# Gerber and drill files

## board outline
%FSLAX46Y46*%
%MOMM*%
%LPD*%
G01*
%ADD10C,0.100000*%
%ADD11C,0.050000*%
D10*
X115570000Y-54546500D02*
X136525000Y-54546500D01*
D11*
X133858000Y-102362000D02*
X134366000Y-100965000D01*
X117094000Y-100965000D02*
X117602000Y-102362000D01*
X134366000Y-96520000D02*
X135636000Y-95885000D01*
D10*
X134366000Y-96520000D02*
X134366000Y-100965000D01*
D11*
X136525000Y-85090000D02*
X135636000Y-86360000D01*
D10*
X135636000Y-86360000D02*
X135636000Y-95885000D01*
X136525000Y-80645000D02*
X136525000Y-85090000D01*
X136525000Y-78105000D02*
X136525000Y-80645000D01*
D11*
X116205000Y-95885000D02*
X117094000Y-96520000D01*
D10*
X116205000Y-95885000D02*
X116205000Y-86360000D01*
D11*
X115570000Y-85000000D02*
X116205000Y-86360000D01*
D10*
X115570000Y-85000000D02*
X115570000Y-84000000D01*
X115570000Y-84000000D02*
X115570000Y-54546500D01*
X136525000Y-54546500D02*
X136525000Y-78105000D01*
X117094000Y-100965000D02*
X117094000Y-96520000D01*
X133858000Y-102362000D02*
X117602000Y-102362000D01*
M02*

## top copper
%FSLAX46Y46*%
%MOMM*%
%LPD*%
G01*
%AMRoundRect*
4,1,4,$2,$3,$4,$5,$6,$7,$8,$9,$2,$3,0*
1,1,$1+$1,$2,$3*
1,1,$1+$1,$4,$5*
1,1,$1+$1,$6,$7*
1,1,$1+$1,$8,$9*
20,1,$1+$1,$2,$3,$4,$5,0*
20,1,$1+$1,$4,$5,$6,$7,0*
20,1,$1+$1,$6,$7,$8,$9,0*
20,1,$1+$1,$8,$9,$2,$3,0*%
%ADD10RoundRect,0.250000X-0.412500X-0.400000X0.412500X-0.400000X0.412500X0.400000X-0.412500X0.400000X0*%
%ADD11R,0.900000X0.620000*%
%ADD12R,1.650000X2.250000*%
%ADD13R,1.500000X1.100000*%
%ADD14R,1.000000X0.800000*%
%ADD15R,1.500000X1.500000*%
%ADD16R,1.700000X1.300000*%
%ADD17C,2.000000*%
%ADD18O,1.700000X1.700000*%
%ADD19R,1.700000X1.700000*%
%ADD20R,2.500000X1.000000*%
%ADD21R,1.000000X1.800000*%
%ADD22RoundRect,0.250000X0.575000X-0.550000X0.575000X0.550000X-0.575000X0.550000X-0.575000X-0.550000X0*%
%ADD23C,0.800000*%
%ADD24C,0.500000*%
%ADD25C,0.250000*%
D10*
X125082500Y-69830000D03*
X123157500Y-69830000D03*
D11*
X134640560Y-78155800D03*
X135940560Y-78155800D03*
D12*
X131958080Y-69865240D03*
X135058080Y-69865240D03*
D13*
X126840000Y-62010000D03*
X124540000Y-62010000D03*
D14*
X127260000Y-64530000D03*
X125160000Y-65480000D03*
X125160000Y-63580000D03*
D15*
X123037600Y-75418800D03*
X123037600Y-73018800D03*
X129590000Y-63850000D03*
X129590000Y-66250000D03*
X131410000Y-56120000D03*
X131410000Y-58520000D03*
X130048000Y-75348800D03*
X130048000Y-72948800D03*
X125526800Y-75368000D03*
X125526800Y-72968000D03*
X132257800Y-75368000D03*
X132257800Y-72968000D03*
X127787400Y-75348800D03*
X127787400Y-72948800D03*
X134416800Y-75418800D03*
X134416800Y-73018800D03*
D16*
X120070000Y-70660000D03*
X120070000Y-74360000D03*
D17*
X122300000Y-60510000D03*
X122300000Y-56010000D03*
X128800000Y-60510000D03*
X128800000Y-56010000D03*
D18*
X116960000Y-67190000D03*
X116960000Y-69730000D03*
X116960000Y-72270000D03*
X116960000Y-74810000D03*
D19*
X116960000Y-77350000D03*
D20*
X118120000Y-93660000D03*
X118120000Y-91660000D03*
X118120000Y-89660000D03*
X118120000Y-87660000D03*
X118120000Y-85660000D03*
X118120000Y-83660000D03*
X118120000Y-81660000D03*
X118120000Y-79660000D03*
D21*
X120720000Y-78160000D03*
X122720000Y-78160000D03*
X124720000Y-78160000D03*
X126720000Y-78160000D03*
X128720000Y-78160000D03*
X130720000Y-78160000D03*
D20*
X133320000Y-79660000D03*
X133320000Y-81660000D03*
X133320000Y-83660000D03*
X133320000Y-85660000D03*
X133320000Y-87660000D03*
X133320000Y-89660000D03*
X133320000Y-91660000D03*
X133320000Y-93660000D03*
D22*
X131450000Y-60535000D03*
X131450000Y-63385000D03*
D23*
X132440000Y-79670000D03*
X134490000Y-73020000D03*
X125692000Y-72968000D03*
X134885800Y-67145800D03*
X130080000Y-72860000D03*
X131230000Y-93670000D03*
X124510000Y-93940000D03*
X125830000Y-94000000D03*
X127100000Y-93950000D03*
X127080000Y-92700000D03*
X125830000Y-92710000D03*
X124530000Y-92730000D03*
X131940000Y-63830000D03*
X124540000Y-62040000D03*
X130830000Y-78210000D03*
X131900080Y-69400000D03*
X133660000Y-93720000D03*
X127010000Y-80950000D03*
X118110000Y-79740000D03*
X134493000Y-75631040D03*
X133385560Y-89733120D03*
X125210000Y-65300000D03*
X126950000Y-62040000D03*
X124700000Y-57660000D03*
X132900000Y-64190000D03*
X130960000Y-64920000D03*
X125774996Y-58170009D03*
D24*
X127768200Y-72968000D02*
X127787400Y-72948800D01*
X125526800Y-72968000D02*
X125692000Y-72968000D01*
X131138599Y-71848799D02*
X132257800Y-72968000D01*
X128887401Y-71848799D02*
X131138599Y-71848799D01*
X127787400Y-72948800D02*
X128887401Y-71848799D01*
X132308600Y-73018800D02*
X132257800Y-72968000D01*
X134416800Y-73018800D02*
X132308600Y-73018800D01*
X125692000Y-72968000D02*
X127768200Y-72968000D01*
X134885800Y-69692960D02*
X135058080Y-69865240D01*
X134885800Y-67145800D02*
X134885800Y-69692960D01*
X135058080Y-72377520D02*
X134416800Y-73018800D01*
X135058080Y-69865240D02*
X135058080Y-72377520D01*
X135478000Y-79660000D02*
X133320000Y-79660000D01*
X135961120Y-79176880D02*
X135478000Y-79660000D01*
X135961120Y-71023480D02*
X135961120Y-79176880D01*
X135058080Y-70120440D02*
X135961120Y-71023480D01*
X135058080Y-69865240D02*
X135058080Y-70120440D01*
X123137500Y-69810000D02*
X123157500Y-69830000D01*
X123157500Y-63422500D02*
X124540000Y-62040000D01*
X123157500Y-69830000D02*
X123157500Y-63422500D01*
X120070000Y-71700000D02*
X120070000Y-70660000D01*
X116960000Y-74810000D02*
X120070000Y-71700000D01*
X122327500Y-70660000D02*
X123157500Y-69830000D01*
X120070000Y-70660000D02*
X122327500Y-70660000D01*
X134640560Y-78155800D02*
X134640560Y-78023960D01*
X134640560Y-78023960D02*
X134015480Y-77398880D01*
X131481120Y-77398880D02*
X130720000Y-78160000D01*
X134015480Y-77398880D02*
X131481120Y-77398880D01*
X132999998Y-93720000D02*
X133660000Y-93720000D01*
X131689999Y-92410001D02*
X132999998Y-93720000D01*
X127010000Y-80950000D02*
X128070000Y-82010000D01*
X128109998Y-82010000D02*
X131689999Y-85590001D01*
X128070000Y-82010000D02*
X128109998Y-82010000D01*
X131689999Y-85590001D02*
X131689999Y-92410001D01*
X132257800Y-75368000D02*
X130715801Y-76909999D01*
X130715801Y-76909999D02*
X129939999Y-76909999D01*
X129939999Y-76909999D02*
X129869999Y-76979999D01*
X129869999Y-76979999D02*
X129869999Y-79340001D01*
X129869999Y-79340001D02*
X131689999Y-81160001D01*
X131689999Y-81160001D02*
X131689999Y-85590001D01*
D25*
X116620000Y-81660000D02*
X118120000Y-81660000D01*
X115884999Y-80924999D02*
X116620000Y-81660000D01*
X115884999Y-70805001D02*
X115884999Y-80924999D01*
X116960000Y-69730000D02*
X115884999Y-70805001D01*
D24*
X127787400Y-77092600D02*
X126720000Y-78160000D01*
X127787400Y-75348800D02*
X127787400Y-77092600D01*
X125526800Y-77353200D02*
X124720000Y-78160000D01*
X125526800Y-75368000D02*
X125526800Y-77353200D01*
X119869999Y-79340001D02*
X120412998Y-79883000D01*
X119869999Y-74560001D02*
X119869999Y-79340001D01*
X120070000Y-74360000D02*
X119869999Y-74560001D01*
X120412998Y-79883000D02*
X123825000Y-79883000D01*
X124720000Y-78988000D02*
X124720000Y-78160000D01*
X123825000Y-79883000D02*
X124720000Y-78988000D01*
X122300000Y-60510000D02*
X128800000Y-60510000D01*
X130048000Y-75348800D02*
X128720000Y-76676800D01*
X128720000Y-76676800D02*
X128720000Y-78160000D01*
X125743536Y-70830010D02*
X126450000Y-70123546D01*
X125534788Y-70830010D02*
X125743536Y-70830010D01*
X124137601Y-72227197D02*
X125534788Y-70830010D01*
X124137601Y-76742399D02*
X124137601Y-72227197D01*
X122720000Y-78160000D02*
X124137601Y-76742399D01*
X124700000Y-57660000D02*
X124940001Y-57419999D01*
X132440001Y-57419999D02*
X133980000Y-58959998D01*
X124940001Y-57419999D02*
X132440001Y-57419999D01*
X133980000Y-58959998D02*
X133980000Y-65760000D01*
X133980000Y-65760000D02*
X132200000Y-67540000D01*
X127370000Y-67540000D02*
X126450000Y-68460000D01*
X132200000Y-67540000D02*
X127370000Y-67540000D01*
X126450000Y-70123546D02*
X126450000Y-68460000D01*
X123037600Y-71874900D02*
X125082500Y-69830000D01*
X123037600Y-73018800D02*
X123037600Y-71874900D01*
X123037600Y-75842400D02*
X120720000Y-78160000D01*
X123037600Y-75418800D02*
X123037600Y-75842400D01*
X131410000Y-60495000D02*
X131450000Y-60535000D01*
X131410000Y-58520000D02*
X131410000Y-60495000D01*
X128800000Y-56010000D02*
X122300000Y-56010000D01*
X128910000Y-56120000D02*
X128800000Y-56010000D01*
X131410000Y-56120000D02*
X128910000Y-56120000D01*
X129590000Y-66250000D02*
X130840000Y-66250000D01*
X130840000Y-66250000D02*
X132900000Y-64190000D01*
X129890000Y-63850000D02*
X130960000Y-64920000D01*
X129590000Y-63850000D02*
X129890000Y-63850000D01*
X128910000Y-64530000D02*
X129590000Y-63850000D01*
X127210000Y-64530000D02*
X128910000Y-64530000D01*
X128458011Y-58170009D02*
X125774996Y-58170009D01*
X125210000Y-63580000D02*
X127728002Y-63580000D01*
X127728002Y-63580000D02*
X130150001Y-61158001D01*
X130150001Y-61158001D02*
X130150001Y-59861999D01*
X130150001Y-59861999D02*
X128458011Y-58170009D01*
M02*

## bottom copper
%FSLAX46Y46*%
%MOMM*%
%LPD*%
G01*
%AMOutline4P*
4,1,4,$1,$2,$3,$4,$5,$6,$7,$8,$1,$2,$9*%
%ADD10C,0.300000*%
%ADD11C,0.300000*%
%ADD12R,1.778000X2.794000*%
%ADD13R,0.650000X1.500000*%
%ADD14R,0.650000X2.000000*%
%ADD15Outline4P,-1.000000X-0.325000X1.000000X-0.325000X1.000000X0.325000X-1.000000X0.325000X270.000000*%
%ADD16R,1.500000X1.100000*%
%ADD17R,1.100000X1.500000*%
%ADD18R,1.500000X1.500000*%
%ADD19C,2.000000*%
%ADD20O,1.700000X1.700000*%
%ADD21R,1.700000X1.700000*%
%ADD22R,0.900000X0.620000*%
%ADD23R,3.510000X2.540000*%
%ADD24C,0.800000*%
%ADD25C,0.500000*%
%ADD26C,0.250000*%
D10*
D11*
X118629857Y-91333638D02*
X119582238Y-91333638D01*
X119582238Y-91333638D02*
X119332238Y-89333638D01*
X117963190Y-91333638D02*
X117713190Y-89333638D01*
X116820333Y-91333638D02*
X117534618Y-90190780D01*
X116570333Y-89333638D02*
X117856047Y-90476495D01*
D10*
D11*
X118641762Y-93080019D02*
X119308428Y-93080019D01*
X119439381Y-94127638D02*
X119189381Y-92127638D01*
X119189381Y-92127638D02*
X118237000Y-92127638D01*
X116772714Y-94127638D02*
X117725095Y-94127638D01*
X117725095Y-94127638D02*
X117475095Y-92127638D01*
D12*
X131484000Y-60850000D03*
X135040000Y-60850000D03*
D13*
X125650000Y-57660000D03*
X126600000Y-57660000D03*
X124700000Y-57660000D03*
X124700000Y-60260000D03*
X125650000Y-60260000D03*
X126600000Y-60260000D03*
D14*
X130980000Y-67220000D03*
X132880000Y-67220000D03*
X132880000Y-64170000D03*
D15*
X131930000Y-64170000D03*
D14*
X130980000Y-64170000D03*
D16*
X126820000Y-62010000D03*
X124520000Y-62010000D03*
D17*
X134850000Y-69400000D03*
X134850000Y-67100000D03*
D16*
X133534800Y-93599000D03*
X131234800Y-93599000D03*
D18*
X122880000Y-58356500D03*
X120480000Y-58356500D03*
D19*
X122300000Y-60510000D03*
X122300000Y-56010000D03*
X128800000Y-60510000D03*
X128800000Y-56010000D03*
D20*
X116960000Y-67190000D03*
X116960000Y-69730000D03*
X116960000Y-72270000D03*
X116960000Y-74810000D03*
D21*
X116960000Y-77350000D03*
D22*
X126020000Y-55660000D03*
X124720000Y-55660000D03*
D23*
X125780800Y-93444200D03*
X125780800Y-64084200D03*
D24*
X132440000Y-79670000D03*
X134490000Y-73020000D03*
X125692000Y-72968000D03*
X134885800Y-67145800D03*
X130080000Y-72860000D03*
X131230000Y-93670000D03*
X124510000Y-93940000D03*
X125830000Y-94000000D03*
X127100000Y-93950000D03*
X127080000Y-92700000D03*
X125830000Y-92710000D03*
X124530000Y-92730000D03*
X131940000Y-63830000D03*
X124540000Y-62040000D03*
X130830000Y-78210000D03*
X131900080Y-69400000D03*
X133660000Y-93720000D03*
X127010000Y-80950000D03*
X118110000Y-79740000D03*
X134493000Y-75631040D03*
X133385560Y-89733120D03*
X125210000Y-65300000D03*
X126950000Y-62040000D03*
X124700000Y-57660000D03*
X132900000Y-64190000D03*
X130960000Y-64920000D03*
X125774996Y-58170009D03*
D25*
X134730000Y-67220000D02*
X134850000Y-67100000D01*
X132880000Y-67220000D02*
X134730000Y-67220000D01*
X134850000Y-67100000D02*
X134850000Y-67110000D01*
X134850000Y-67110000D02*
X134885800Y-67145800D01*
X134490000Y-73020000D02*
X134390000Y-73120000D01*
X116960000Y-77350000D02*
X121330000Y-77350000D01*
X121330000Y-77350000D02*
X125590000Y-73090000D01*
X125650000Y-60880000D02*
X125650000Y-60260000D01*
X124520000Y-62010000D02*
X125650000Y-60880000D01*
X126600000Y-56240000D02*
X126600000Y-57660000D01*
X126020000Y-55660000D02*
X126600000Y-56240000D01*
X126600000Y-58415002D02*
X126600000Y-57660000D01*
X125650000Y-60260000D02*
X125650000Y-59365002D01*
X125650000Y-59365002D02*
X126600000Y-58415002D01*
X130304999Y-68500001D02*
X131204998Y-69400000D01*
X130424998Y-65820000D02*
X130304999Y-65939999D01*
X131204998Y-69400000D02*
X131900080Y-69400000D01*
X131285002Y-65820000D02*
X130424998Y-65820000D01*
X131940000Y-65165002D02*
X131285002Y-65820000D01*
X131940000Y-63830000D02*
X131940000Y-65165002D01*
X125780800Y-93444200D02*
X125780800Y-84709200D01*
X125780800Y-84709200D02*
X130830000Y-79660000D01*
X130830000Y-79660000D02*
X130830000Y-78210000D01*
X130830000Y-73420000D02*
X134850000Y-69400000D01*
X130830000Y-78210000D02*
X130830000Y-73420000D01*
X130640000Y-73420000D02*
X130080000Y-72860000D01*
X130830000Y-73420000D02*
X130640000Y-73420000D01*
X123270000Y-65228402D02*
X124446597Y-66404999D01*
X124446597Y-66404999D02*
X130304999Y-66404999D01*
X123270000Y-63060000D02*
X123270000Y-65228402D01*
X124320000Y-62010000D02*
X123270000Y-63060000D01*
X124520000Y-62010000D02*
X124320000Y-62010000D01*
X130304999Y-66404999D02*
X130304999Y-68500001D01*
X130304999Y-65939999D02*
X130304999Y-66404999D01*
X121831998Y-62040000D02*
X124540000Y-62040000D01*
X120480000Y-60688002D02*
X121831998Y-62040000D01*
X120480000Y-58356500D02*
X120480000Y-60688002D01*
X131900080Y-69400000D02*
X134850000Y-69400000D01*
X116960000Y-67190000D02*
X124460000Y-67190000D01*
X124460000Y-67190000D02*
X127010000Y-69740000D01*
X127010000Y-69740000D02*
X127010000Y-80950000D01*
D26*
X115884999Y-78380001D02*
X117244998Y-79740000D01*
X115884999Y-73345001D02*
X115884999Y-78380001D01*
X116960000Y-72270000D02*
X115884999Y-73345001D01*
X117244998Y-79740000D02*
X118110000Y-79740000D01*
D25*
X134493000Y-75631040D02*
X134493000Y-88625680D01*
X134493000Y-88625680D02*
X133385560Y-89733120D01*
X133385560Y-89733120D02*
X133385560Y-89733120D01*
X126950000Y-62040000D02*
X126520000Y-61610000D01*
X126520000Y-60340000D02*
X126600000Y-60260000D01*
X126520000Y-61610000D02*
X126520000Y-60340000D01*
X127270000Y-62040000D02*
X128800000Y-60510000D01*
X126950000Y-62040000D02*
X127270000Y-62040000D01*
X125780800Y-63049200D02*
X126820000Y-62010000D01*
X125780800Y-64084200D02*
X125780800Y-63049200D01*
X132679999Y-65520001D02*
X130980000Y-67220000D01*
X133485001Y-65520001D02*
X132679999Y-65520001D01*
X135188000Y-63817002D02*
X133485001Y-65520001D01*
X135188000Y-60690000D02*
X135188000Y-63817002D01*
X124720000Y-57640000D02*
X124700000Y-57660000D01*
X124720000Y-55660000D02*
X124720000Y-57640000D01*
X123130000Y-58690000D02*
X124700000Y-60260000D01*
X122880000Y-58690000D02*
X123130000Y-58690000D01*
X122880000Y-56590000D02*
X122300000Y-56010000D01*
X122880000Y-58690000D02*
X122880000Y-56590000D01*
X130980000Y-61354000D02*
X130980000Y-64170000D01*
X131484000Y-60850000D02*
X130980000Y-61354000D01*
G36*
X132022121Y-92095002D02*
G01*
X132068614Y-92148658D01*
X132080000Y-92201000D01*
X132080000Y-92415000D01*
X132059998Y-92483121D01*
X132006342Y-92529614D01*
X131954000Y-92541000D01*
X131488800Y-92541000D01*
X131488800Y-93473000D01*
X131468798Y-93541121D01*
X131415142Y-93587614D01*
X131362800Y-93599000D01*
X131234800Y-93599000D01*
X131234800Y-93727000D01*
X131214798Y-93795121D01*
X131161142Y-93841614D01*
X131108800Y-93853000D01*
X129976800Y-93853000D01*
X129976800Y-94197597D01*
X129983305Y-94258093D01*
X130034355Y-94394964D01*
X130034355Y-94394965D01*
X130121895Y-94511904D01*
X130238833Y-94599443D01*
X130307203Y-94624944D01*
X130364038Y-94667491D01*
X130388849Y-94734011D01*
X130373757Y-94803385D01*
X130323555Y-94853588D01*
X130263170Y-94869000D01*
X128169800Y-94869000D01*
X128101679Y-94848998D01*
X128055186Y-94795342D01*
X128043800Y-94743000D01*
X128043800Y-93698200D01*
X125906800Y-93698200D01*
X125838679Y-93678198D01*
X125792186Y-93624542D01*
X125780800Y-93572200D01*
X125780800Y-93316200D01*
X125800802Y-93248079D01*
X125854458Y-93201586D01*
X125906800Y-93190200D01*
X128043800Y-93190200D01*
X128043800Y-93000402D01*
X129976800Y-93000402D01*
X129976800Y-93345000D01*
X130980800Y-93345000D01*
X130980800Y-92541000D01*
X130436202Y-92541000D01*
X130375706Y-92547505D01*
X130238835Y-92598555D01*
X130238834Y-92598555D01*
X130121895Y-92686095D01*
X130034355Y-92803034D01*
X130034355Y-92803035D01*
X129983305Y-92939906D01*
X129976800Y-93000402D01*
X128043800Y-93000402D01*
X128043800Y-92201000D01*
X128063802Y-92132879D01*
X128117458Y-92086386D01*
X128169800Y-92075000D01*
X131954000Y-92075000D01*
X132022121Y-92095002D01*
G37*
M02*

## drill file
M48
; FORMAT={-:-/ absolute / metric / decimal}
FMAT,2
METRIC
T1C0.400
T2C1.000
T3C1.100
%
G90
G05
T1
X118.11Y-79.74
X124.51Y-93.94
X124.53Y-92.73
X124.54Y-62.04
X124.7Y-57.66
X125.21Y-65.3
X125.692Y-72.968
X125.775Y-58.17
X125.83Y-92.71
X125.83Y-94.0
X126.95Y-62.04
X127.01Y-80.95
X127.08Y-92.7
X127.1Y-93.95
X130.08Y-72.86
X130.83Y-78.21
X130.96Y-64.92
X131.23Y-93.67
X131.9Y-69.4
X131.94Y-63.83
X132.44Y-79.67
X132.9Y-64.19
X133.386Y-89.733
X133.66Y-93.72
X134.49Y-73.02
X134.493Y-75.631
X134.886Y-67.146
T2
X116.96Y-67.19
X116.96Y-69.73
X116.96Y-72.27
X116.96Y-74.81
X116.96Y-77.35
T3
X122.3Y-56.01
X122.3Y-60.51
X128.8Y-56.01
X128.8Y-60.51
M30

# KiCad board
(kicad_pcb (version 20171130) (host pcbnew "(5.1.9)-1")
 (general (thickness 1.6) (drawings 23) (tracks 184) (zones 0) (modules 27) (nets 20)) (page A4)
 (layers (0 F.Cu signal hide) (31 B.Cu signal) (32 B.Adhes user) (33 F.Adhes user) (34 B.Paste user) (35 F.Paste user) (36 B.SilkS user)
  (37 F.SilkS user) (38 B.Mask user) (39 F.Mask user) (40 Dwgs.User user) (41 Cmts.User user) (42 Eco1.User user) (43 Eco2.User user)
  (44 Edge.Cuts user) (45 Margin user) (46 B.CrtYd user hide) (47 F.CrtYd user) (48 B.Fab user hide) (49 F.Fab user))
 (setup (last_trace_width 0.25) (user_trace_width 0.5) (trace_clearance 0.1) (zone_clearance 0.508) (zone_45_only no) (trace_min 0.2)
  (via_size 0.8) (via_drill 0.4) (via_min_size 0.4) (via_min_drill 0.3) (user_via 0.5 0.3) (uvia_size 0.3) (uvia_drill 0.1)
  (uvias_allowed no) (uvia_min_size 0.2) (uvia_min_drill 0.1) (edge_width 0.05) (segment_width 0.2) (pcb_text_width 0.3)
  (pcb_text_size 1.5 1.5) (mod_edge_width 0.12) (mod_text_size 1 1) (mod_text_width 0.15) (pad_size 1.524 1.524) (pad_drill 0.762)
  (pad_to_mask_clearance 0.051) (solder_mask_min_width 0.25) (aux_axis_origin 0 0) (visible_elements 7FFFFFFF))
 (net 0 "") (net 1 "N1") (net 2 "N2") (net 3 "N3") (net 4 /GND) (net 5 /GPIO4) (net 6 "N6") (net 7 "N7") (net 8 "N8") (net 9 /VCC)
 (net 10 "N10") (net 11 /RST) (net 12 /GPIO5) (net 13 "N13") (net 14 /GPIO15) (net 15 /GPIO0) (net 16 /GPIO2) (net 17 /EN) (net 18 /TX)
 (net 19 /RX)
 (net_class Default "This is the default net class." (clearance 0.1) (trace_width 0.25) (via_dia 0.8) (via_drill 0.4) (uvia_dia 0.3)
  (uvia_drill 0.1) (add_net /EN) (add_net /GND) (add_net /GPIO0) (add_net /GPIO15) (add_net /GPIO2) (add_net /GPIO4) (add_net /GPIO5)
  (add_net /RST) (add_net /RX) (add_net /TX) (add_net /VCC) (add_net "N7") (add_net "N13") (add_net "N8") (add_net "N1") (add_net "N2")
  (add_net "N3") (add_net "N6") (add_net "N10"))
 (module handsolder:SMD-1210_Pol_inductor (layer B.Cu) (at 133.262 60.85)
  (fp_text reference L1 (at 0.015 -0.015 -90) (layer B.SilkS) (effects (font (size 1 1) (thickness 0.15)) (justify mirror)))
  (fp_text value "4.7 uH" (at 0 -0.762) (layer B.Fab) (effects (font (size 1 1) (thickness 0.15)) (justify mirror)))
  (pad 1 smd rect (at -1.778 0) (size 1.778 2.794) (layers B.Cu B.Paste B.Mask) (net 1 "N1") (zone_connect 2))
  (pad 2 smd rect (at 1.778 0) (size 1.778 2.794) (layers B.Cu B.Paste B.Mask) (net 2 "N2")))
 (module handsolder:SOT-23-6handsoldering (layer B.Cu) (at 125.65 58.96 90)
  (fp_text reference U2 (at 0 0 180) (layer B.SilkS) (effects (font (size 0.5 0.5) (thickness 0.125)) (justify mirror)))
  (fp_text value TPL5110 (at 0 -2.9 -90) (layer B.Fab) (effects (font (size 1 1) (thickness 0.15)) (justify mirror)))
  (pad 5 smd rect (at 1.3 0 90) (size 1.5 0.65) (layers B.Cu B.Paste B.Mask) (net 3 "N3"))
  (pad 6 smd rect (at 1.3 0.95 90) (size 1.5 0.65) (layers B.Cu B.Paste B.Mask) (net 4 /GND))
  (pad 4 smd rect (at 1.3 -0.95 90) (size 1.5 0.65) (layers B.Cu B.Paste B.Mask) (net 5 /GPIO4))
  (pad 3 smd rect (at -1.3 -0.95 90) (size 1.5 0.65) (layers B.Cu B.Paste B.Mask) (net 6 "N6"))
  (pad 2 smd rect (at -1.3 0 90) (size 1.5 0.65) (layers B.Cu B.Paste B.Mask) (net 4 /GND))
  (pad 1 smd rect (at -1.3 0.95 90) (size 1.5 0.65) (layers B.Cu B.Paste B.Mask) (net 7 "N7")))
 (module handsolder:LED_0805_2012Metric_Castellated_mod (layer F.Cu) (at 124.12 69.83)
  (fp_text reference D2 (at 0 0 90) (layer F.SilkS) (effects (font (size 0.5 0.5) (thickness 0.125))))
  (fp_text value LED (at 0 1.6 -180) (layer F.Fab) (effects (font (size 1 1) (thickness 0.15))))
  (pad 2 smd roundrect (at 0.9625 0) (size 1.325 1.3) (layers F.Cu F.Paste F.Mask) (roundrect_rratio 0.1923076923076923) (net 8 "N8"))
  (pad 1 smd roundrect (at -0.9625 0) (size 1.325 1.3) (layers F.Cu F.Paste F.Mask) (roundrect_rratio 0.1923076923076923) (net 4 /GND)))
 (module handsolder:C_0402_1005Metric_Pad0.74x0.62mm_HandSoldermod (layer F.Cu) (at 135.29056 78.1558 180)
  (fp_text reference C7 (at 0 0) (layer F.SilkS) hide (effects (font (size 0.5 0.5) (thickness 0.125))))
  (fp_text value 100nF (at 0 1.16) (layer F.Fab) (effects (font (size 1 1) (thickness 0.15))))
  (pad 2 smd rect (at 0.65 0 180) (size 0.9 0.62) (layers F.Cu F.Paste F.Mask) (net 4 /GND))
  (pad 1 smd rect (at -0.65 0 180) (size 0.9 0.62) (layers F.Cu F.Paste F.Mask) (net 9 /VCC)))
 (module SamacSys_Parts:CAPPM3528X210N (layer F.Cu) (at 133.50808 69.86524 180)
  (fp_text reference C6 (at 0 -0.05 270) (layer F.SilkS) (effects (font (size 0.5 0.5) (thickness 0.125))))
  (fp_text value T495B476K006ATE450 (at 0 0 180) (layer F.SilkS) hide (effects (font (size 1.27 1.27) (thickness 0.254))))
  (pad 2 smd rect (at 1.55 0 180) (size 1.65 2.25) (layers F.Cu F.Paste F.Mask) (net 4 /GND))
  (pad 1 smd rect (at -1.55 0 180) (size 1.65 2.25) (layers F.Cu F.Paste F.Mask) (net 9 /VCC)))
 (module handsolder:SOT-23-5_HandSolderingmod (layer B.Cu) (at 131.93 65.72 270)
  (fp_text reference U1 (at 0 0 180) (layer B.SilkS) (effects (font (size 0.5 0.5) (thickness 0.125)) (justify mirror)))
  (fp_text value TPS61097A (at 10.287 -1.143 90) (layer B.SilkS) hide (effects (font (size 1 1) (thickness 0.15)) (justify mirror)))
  (pad 5 smd rect (at 1.5 0.95 270) (size 2 0.65) (layers B.Cu B.Paste B.Mask) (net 2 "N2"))
  (pad 4 smd rect (at 1.5 -0.95 270) (size 2 0.65) (layers B.Cu B.Paste B.Mask) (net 9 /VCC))
  (pad 3 smd rect (at -1.55 -0.95 270) (size 2 0.65) (layers B.Cu B.Paste B.Mask) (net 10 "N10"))
  (pad 2 smd trapezoid (at -1.55 0 270) (size 2 0.65) (layers B.Cu B.Paste B.Mask) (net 4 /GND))
  (pad 1 smd rect (at -1.55 0.95 270) (size 2 0.65) (layers B.Cu B.Paste B.Mask) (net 1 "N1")))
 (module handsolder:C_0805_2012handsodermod (layer F.Cu) (at 125.69 62.01)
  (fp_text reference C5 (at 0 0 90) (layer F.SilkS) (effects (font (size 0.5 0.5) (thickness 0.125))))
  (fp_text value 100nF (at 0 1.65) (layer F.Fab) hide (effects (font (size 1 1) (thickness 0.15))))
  (pad 2 smd rect (at 1.15 0) (size 1.5 1.1) (layers F.Cu F.Paste F.Mask) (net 7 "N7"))
  (pad 1 smd rect (at -1.15 0) (size 1.5 1.1) (layers F.Cu F.Paste F.Mask) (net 4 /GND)))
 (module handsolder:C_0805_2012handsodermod (layer B.Cu) (at 125.67 62.01)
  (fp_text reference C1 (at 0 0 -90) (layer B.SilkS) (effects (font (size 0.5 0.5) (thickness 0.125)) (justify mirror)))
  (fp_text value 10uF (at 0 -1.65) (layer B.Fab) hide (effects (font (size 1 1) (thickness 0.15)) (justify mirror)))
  (pad 2 smd rect (at 1.15 0) (size 1.5 1.1) (layers B.Cu B.Paste B.Mask) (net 7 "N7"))
  (pad 1 smd rect (at -1.15 0) (size 1.5 1.1) (layers B.Cu B.Paste B.Mask) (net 4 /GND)))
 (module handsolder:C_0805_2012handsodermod (layer B.Cu) (at 134.85 68.25 270)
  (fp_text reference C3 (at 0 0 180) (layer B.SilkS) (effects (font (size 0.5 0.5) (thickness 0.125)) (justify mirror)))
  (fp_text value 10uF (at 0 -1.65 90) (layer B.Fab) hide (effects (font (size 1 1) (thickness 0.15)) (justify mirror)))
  (pad 2 smd rect (at 1.15 0 270) (size 1.5 1.1) (layers B.Cu B.Paste B.Mask) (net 4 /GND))
  (pad 1 smd rect (at -1.15 0 270) (size 1.5 1.1) (layers B.Cu B.Paste B.Mask) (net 9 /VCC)))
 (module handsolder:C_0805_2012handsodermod (layer B.Cu) (at 132.3848 93.599)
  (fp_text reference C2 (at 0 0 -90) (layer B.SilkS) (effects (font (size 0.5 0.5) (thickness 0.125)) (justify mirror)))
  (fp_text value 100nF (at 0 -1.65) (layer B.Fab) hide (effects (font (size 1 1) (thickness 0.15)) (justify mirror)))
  (pad 2 smd rect (at 1.15 0) (size 1.5 1.1) (layers B.Cu B.Paste B.Mask) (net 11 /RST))
  (pad 1 smd rect (at -1.15 0) (size 1.5 1.1) (layers B.Cu B.Paste B.Mask) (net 4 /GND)))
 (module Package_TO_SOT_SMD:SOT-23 (layer F.Cu) (at 126.21 64.53)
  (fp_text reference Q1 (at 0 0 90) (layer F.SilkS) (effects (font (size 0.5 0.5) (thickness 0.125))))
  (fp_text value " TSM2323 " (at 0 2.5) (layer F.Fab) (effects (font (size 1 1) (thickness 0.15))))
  (pad 3 smd rect (at 1.05 0) (size 1 0.8) (layers F.Cu F.Paste F.Mask) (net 1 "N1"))
  (pad 2 smd rect (at -1.05 0.95) (size 1 0.8) (layers F.Cu F.Paste F.Mask) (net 7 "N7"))
  (pad 1 smd rect (at -1.05 -0.95) (size 1 0.8) (layers F.Cu F.Paste F.Mask) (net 3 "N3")))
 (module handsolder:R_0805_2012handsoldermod (layer F.Cu) (at 123.0376 74.2188 270)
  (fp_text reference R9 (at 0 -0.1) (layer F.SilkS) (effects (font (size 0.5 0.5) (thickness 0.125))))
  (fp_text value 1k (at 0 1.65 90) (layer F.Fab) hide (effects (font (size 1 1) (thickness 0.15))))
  (pad 2 smd rect (at 1.2 0 270) (size 1.5 1.5) (layers F.Cu F.Paste F.Mask) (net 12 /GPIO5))
  (pad 1 smd rect (at -1.2 0 270) (size 1.5 1.5) (layers F.Cu F.Paste F.Mask) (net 8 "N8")))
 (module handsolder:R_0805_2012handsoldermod (layer B.Cu) (at 121.68 58.3565)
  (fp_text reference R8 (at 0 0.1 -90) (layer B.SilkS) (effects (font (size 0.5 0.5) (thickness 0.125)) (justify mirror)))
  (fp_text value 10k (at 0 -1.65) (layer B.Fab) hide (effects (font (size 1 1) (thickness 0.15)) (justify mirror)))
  (pad 2 smd rect (at 1.2 0) (size 1.5 1.5) (layers B.Cu B.Paste B.Mask) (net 6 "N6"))
  (pad 1 smd rect (at -1.2 0) (size 1.5 1.5) (layers B.Cu B.Paste B.Mask) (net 4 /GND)))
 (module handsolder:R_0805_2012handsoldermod (layer F.Cu) (at 129.59 65.05 90)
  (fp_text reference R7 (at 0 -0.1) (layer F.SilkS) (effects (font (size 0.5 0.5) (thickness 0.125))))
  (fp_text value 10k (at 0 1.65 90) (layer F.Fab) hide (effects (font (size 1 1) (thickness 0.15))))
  (pad 2 smd rect (at 1.2 0 90) (size 1.5 1.5) (layers F.Cu F.Paste F.Mask) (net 1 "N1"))
  (pad 1 smd rect (at -1.2 0 90) (size 1.5 1.5) (layers F.Cu F.Paste F.Mask) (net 10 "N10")))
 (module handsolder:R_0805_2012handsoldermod (layer F.Cu) (at 131.41 57.32 90)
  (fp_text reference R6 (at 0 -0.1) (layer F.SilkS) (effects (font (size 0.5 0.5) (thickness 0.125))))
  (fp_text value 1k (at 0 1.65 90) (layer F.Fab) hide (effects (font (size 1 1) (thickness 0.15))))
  (pad 2 smd rect (at 1.2 0 90) (size 1.5 1.5) (layers F.Cu F.Paste F.Mask) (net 6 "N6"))
  (pad 1 smd rect (at -1.2 0 90) (size 1.5 1.5) (layers F.Cu F.Paste F.Mask) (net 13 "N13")))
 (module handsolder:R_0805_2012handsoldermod (layer F.Cu) (at 130.048 74.1488 270)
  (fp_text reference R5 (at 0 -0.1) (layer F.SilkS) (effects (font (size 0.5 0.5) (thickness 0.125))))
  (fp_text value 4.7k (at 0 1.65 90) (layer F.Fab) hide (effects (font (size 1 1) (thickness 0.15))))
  (pad 2 smd rect (at 1.2 0 270) (size 1.5 1.5) (layers F.Cu F.Paste F.Mask) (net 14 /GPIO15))
  (pad 1 smd rect (at -1.2 0 270) (size 1.5 1.5) (layers F.Cu F.Paste F.Mask) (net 4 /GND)))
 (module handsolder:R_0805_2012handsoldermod (layer F.Cu) (at 125.5268 74.168 270)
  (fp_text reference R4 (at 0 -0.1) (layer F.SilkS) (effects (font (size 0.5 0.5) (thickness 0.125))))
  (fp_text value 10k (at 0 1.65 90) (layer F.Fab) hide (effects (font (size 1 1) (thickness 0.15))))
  (pad 2 smd rect (at 1.2 0 270) (size 1.5 1.5) (layers F.Cu F.Paste F.Mask) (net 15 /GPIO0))
  (pad 1 smd rect (at -1.2 0 270) (size 1.5 1.5) (layers F.Cu F.Paste F.Mask) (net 9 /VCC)))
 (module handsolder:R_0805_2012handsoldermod (layer F.Cu) (at 132.2578 74.168 270)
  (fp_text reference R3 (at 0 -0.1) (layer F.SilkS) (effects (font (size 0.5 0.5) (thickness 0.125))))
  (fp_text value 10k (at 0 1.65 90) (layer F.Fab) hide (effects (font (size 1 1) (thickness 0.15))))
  (pad 2 smd rect (at 1.2 0 270) (size 1.5 1.5) (layers F.Cu F.Paste F.Mask) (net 11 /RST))
  (pad 1 smd rect (at -1.2 0 270) (size 1.5 1.5) (layers F.Cu F.Paste F.Mask) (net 9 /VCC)))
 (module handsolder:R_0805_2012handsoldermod (layer F.Cu) (at 127.7874 74.1488 270)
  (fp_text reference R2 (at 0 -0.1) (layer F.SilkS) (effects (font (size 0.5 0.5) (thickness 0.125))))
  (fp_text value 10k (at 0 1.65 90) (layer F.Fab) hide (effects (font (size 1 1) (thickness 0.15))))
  (pad 2 smd rect (at 1.2 0 270) (size 1.5 1.5) (layers F.Cu F.Paste F.Mask) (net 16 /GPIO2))
  (pad 1 smd rect (at -1.2 0 270) (size 1.5 1.5) (layers F.Cu F.Paste F.Mask) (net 9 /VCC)))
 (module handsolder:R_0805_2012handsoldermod (layer F.Cu) (at 134.4168 74.2188 270)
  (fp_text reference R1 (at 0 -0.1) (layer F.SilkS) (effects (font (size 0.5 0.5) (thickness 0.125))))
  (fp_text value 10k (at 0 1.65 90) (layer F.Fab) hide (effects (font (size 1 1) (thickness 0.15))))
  (pad 2 smd rect (at 1.2 0 270) (size 1.5 1.5) (layers F.Cu F.Paste F.Mask) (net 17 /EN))
  (pad 1 smd rect (at -1.2 0 270) (size 1.5 1.5) (layers F.Cu F.Paste F.Mask) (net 9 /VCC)))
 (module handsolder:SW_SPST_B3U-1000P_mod (layer F.Cu) (at 120.07 72.51 90)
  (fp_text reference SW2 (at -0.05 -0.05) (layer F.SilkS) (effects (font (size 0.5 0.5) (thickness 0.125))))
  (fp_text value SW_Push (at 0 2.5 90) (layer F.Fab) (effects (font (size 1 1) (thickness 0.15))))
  (pad 2 smd rect (at 1.85 0 90) (size 1.3 1.7) (layers F.Cu F.Paste F.Mask) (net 4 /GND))
  (pad 1 smd rect (at -1.85 0 90) (size 1.3 1.7) (layers F.Cu F.Paste F.Mask) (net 15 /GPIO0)))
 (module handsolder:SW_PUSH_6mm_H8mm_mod (layer F.Cu) (at 128.8 60.51 180)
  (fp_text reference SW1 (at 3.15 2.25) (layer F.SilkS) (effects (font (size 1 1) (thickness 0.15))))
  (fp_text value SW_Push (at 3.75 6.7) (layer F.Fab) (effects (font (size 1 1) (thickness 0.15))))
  (pad 1 thru_hole circle (at 6.5 0 270) (size 2 2) (drill 1.1) (layers *.Cu *.Mask) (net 7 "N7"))
  (pad 2 thru_hole circle (at 6.5 4.5 270) (size 2 2) (drill 1.1) (layers *.Cu *.Mask) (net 6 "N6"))
  (pad 1 thru_hole circle (at 0 0 270) (size 2 2) (drill 1.1) (layers *.Cu *.Mask) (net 7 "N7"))
  (pad 2 thru_hole circle (at 0 4.5 270) (size 2 2) (drill 1.1) (layers *.Cu *.Mask) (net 6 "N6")))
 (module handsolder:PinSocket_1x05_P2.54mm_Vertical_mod (layer F.Cu) (at 116.96 77.35 180)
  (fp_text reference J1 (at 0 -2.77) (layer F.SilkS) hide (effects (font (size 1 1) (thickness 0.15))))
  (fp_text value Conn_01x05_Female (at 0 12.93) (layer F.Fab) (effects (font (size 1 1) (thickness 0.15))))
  (pad 5 thru_hole oval (at 0 10.16 180) (size 1.7 1.7) (drill 1) (layers *.Cu *.Mask) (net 11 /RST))
  (pad 4 thru_hole oval (at 0 7.62 180) (size 1.7 1.7) (drill 1) (layers *.Cu *.Mask) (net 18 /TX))
  (pad 3 thru_hole oval (at 0 5.08 180) (size 1.7 1.7) (drill 1) (layers *.Cu *.Mask) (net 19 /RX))
  (pad 2 thru_hole oval (at 0 2.54 180) (size 1.7 1.7) (drill 1) (layers *.Cu *.Mask) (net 4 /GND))
  (pad 1 thru_hole rect (at 0 0 180) (size 1.7 1.7) (drill 1) (layers *.Cu *.Mask) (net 9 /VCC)))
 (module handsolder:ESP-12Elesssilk (layer F.Cu) (at 125.72 90.16 180)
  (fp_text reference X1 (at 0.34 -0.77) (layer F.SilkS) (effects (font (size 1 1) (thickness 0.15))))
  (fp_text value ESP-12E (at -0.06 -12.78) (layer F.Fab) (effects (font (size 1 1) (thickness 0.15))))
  (pad 22 smd rect (at 7.6 -3.5 180) (size 2.5 1) (layers F.Cu F.Paste F.Mask))
  (pad 21 smd rect (at 7.6 -1.5 180) (size 2.5 1) (layers F.Cu F.Paste F.Mask))
  (pad 20 smd rect (at 7.6 0.5 180) (size 2.5 1) (layers F.Cu F.Paste F.Mask))
  (pad 19 smd rect (at 7.6 2.5 180) (size 2.5 1) (layers F.Cu F.Paste F.Mask))
  (pad 18 smd rect (at 7.6 4.5 180) (size 2.5 1) (layers F.Cu F.Paste F.Mask))
  (pad 17 smd rect (at 7.6 6.5 180) (size 2.5 1) (layers F.Cu F.Paste F.Mask))
  (pad 16 smd rect (at 7.6 8.5 180) (size 2.5 1) (layers F.Cu F.Paste F.Mask) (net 18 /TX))
  (pad 15 smd rect (at 7.6 10.5 180) (size 2.5 1) (layers F.Cu F.Paste F.Mask) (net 19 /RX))
  (pad 14 smd rect (at 5 12 180) (size 1 1.8) (layers F.Cu F.Paste F.Mask) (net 12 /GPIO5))
  (pad 13 smd rect (at 3 12 180) (size 1 1.8) (layers F.Cu F.Paste F.Mask) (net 5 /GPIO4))
  (pad 12 smd rect (at 1 12 180) (size 1 1.8) (layers F.Cu F.Paste F.Mask) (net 15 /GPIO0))
  (pad 11 smd rect (at -1 12 180) (size 1 1.8) (layers F.Cu F.Paste F.Mask) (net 16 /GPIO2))
  (pad 10 smd rect (at -3 12 180) (size 1 1.8) (layers F.Cu F.Paste F.Mask) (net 14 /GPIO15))
  (pad 9 smd rect (at -5 12 180) (size 1 1.8) (layers F.Cu F.Paste F.Mask) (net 4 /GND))
  (pad 8 smd rect (at -7.6 10.5 180) (size 2.5 1) (layers F.Cu F.Paste F.Mask) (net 9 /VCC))
  (pad 7 smd rect (at -7.6 8.5 180) (size 2.5 1) (layers F.Cu F.Paste F.Mask))
  (pad 6 smd rect (at -7.6 6.5 180) (size 2.5 1) (layers F.Cu F.Paste F.Mask))
  (pad 5 smd rect (at -7.6 4.5 180) (size 2.5 1) (layers F.Cu F.Paste F.Mask))
  (pad 4 smd rect (at -7.6 2.5 180) (size 2.5 1) (layers F.Cu F.Paste F.Mask))
  (pad 3 smd rect (at -7.6 0.5 180) (size 2.5 1) (layers F.Cu F.Paste F.Mask) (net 17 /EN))
  (pad 2 smd rect (at -7.6 -1.5 180) (size 2.5 1) (layers F.Cu F.Paste F.Mask))
  (pad 1 smd rect (at -7.6 -3.5 180) (size 2.5 1) (layers F.Cu F.Paste F.Mask) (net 11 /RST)))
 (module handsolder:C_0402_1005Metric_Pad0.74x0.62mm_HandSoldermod (layer B.Cu) (at 125.37 55.66)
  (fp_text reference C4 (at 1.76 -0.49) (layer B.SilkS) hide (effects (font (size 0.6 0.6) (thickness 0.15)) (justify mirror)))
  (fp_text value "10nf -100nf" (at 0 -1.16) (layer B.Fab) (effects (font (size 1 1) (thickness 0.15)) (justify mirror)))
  (pad 2 smd rect (at 0.65 0) (size 0.9 0.62) (layers B.Cu B.Paste B.Mask) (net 4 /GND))
  (pad 1 smd rect (at -0.65 0) (size 0.9 0.62) (layers B.Cu B.Paste B.Mask) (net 5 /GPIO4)))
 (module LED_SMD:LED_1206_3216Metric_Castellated (layer F.Cu) (at 131.45 61.96 90)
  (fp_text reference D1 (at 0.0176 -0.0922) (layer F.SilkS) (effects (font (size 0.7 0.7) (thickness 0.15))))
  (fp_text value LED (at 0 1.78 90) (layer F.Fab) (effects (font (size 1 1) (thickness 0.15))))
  (pad 2 smd roundrect (at 1.425 0 90) (size 1.6 1.65) (layers F.Cu F.Paste F.Mask) (roundrect_rratio 0.15625) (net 13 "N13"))
  (pad 1 smd roundrect (at -1.425 0 90) (size 1.6 1.65) (layers F.Cu F.Paste F.Mask) (roundrect_rratio 0.15625) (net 4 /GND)))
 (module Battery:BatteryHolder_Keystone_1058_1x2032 (layer B.Cu) (at 125.7808 78.7642 270)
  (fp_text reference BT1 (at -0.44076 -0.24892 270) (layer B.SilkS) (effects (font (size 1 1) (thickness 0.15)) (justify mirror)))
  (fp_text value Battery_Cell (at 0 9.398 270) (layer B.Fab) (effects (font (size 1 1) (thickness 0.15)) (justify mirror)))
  (pad 2 smd rect (at 14.68 0 270) (size 2.54 3.51) (layers B.Cu B.Paste B.Mask) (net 4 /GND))
  (pad 1 smd rect (at -14.68 0 270) (size 2.54 3.51) (layers B.Cu B.Paste B.Mask) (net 7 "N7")))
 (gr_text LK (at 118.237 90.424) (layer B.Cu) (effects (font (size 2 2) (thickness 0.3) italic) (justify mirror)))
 (gr_line (start 115.57 54.5465) (end 136.525 54.5465) (layer Edge.Cuts) (width 0.1))
 (gr_line (start 133.858 102.362) (end 134.366 100.965) (layer Edge.Cuts) (width 0.05))
 (gr_line (start 117.094 100.965) (end 117.602 102.362) (layer Edge.Cuts) (width 0.05))
 (gr_line (start 134.366 96.52) (end 135.636 95.885) (layer Edge.Cuts) (width 0.05))
 (gr_line (start 134.366 96.52) (end 134.366 100.965) (layer Edge.Cuts) (width 0.1))
 (gr_line (start 136.525 85.09) (end 135.636 86.36) (layer Edge.Cuts) (width 0.05))
 (gr_line (start 135.636 86.36) (end 135.636 95.885) (layer Edge.Cuts) (width 0.1))
 (gr_line (start 136.525 80.645) (end 136.525 85.09) (layer Edge.Cuts) (width 0.1))
 (gr_line (start 136.525 78.105) (end 136.525 80.645) (layer Edge.Cuts) (width 0.1))
 (gr_line (start 116.205 95.885) (end 117.094 96.52) (layer Edge.Cuts) (width 0.05))
 (gr_line (start 116.205 95.885) (end 116.205 86.36) (layer Edge.Cuts) (width 0.1))
 (gr_line (start 115.57 85) (end 116.205 86.36) (layer Edge.Cuts) (width 0.05))
 (gr_line (start 115.57 85) (end 115.57 84) (layer Edge.Cuts) (width 0.1))
 (gr_line (start 115.57 84) (end 115.57 54.5465) (layer Edge.Cuts) (width 0.1))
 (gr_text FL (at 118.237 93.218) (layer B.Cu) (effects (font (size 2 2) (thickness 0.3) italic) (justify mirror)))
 (gr_line (start 136.525 54.5465) (end 136.525 78.105) (layer Edge.Cuts) (width 0.1))
 (gr_line (start 117.094 100.965) (end 117.094 96.52) (layer Edge.Cuts) (width 0.1))
 (gr_line (start 133.858 102.362) (end 117.602 102.362) (layer Edge.Cuts) (width 0.1))
 (via (at 132.44 79.67) (size 0.8) (drill 0.4) (layers F.Cu B.Cu) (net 9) (status 30))
 (segment (start 134.73 67.22) (end 134.85 67.1) (width 0.5) (layer B.Cu) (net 9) (status 30))
 (segment (start 132.88 67.22) (end 134.73 67.22) (width 0.5) (layer B.Cu) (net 9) (status 30))
 (segment (start 127.7682 72.968) (end 127.7874 72.9488) (width 0.5) (layer F.Cu) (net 9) (status 30))
 (segment (start 125.5268 72.968) (end 125.692 72.968) (width 0.5) (layer F.Cu) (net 9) (status 30))
 (segment (start 131.138599 71.848799) (end 132.2578 72.968) (width 0.5) (layer F.Cu) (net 9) (status 20))
 (segment (start 128.887401 71.848799) (end 131.138599 71.848799) (width 0.5) (layer F.Cu) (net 9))
 (segment (start 127.7874 72.9488) (end 128.887401 71.848799) (width 0.5) (layer F.Cu) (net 9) (status 10))
 (segment (start 132.3086 73.0188) (end 132.2578 72.968) (width 0.5) (layer F.Cu) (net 9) (status 30))
 (segment (start 134.4168 73.0188) (end 132.3086 73.0188) (width 0.5) (layer F.Cu) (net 9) (status 30))
 (segment (start 134.85 67.1) (end 134.85 67.11) (width 0.5) (layer B.Cu) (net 9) (status 30))
 (segment (start 134.85 67.11) (end 134.8858 67.1458) (width 0.5) (layer B.Cu) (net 9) (status 10))
 (segment (start 134.49 73.02) (end 134.39 73.12) (width 0.5) (layer B.Cu) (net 9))
 (via (at 134.49 73.02) (size 0.8) (drill 0.4) (layers F.Cu B.Cu) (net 9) (status 30))
 (segment (start 116.96 77.35) (end 121.33 77.35) (width 0.5) (layer B.Cu) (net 9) (status 10))
 (segment (start 121.33 77.35) (end 125.59 73.09) (width 0.5) (layer B.Cu) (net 9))
 (segment (start 125.692 72.968) (end 127.7682 72.968) (width 0.5) (layer F.Cu) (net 9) (status 30))
 (via (at 125.692 72.968) (size 0.8) (drill 0.4) (layers F.Cu B.Cu) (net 9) (status 30))
 (via (at 134.8858 67.1458) (size 0.8) (drill 0.4) (layers F.Cu B.Cu) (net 9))
 (segment (start 134.8858 69.69296) (end 135.05808 69.86524) (width 0.5) (layer F.Cu) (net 9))
 (segment (start 134.8858 67.1458) (end 134.8858 69.69296) (width 0.5) (layer F.Cu) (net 9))
 (segment (start 135.05808 72.37752) (end 134.4168 73.0188) (width 0.5) (layer F.Cu) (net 9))
 (segment (start 135.05808 69.86524) (end 135.05808 72.37752) (width 0.5) (layer F.Cu) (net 9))
 (segment (start 135.478 79.66) (end 133.32 79.66) (width 0.5) (layer F.Cu) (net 9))
 (segment (start 135.96112 79.17688) (end 135.478 79.66) (width 0.5) (layer F.Cu) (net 9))
 (segment (start 135.96112 71.02348) (end 135.96112 79.17688) (width 0.5) (layer F.Cu) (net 9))
 (segment (start 135.05808 70.12044) (end 135.96112 71.02348) (width 0.5) (layer F.Cu) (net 9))
 (segment (start 135.05808 69.86524) (end 135.05808 70.12044) (width 0.5) (layer F.Cu) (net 9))
 (via (at 130.08 72.86) (size 0.8) (drill 0.4) (layers F.Cu B.Cu) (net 4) (status 30))
 (via (at 131.23 93.67) (size 0.8) (drill 0.4) (layers F.Cu B.Cu) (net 4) (status 30))
 (via (at 124.51 93.94) (size 0.8) (drill 0.4) (layers F.Cu B.Cu) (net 4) (status 30))
 (via (at 125.83 94) (size 0.8) (drill 0.4) (layers F.Cu B.Cu) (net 4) (status 30))
 (via (at 127.1 93.95) (size 0.8) (drill 0.4) (layers F.Cu B.Cu) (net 4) (status 30))
 (via (at 127.08 92.7) (size 0.8) (drill 0.4) (layers F.Cu B.Cu) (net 4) (status 30))
 (via (at 125.83 92.71) (size 0.8) (drill 0.4) (layers F.Cu B.Cu) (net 4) (status 30))
 (via (at 124.53 92.73) (size 0.8) (drill 0.4) (layers F.Cu B.Cu) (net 4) (status 30))
 (via (at 131.94 63.83) (size 0.8) (drill 0.4) (layers F.Cu B.Cu) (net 4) (status 30))
 (via (at 124.54 62.04) (size 0.8) (drill 0.4) (layers F.Cu B.Cu) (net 4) (status 30))
 (segment (start 125.65 60.88) (end 125.65 60.26) (width 0.5) (layer B.Cu) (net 4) (status 20))
 (segment (start 124.52 62.01) (end 125.65 60.88) (width 0.5) (layer B.Cu) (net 4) (status 10))
 (segment (start 126.6 56.24) (end 126.6 57.66) (width 0.5) (layer B.Cu) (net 4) (status 20))
 (segment (start 126.02 55.66) (end 126.6 56.24) (width 0.5) (layer B.Cu) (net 4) (status 10))
 (segment (start 126.6 58.415002) (end 126.6 57.66) (width 0.5) (layer B.Cu) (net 4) (status 20))
 (segment (start 125.65 60.26) (end 125.65 59.365002) (width 0.5) (layer B.Cu) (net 4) (status 10))
 (segment (start 125.65 59.365002) (end 126.6 58.415002) (width 0.5) (layer B.Cu) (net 4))
 (segment (start 130.304999 68.500001) (end 131.204998 69.4) (width 0.5) (layer B.Cu) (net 4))
 (segment (start 130.424998 65.82) (end 130.304999 65.939999) (width 0.5) (layer B.Cu) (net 4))
 (segment (start 131.204998 69.4) (end 131.90008 69.4) (width 0.5) (layer B.Cu) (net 4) (status 20))
 (segment (start 131.285002 65.82) (end 130.424998 65.82) (width 0.5) (layer B.Cu) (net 4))
 (segment (start 131.94 65.165002) (end 131.285002 65.82) (width 0.5) (layer B.Cu) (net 4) (status 10))
 (segment (start 131.94 63.83) (end 131.94 65.165002) (width 0.5) (layer B.Cu) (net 4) (status 30))
 (segment (start 125.7808 93.4442) (end 125.7808 84.7092) (width 0.5) (layer B.Cu) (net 4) (status 10))
 (segment (start 125.7808 84.7092) (end 130.83 79.66) (width 0.5) (layer B.Cu) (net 4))
 (segment (start 130.83 79.66) (end 130.83 78.21) (width 0.5) (layer B.Cu) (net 4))
 (via (at 130.83 78.21) (size 0.8) (drill 0.4) (layers F.Cu B.Cu) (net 4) (status 30))
 (segment (start 130.83 73.42) (end 134.85 69.4) (width 0.5) (layer B.Cu) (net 4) (status 20))
 (segment (start 130.83 78.21) (end 130.83 73.42) (width 0.5) (layer B.Cu) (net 4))
 (segment (start 130.64 73.42) (end 130.08 72.86) (width 0.5) (layer B.Cu) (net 4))
 (segment (start 130.83 73.42) (end 130.64 73.42) (width 0.5) (layer B.Cu) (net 4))
 (segment (start 123.1375 69.81) (end 123.1575 69.83) (width 0.5) (layer F.Cu) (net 4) (status 30))
 (segment (start 123.1575 63.4225) (end 124.54 62.04) (width 0.5) (layer F.Cu) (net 4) (status 20))
 (segment (start 123.1575 69.83) (end 123.1575 63.4225) (width 0.5) (layer F.Cu) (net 4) (status 10))
 (segment (start 123.27 65.228402) (end 124.446597 66.404999) (width 0.5) (layer B.Cu) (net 4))
 (segment (start 124.446597 66.404999) (end 130.304999 66.404999) (width 0.5) (layer B.Cu) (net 4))
 (segment (start 123.27 63.06) (end 123.27 65.228402) (width 0.5) (layer B.Cu) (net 4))
 (segment (start 124.32 62.01) (end 123.27 63.06) (width 0.5) (layer B.Cu) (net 4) (status 10))
 (segment (start 124.52 62.01) (end 124.32 62.01) (width 0.5) (layer B.Cu) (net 4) (status 30))
 (segment (start 130.304999 66.404999) (end 130.304999 68.500001) (width 0.5) (layer B.Cu) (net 4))
 (segment (start 130.304999 65.939999) (end 130.304999 66.404999) (width 0.5) (layer B.Cu) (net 4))
 (segment (start 120.07 71.7) (end 120.07 70.66) (width 0.5) (layer F.Cu) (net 4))
 (segment (start 116.96 74.81) (end 120.07 71.7) (width 0.5) (layer F.Cu) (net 4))
 (segment (start 122.3275 70.66) (end 123.1575 69.83) (width 0.5) (layer F.Cu) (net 4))
 (segment (start 120.07 70.66) (end 122.3275 70.66) (width 0.5) (layer F.Cu) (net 4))
 (segment (start 121.831998 62.04) (end 124.54 62.04) (width 0.5) (layer B.Cu) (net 4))
 (segment (start 120.48 60.688002) (end 121.831998 62.04) (width 0.5) (layer B.Cu) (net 4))
 (segment (start 120.48 58.3565) (end 120.48 60.688002) (width 0.5) (layer B.Cu) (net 4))
 (segment (start 131.90008 69.4) (end 134.85 69.4) (width 0.5) (layer B.Cu) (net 4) (status 20))
 (via (at 131.90008 69.4) (size 0.8) (drill 0.4) (layers F.Cu B.Cu) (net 4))
 (segment (start 134.64056 78.1558) (end 134.64056 78.02396) (width 0.5) (layer F.Cu) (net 4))
 (segment (start 134.64056 78.02396) (end 134.01548 77.39888) (width 0.5) (layer F.Cu) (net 4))
 (segment (start 131.48112 77.39888) (end 130.72 78.16) (width 0.5) (layer F.Cu) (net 4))
 (segment (start 134.01548 77.39888) (end 131.48112 77.39888) (width 0.5) (layer F.Cu) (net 4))
 (via (at 133.66 93.72) (size 0.8) (drill 0.4) (layers F.Cu B.Cu) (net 11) (status 30))
 (segment (start 132.999998 93.72) (end 133.66 93.72) (width 0.5) (layer F.Cu) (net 11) (status 30))
 (segment (start 131.689999 92.410001) (end 132.999998 93.72) (width 0.5) (layer F.Cu) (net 11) (status 20))
 (segment (start 116.96 67.19) (end 124.46 67.19) (width 0.5) (layer B.Cu) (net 11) (status 10))
 (segment (start 124.46 67.19) (end 127.01 69.74) (width 0.5) (layer B.Cu) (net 11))
 (segment (start 127.01 69.74) (end 127.01 80.95) (width 0.5) (layer B.Cu) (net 11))
 (via (at 127.01 80.95) (size 0.8) (drill 0.4) (layers F.Cu B.Cu) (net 11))
 (segment (start 127.01 80.95) (end 128.07 82.01) (width 0.5) (layer F.Cu) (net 11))
 (segment (start 128.109998 82.01) (end 131.689999 85.590001) (width 0.5) (layer F.Cu) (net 11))
 (segment (start 128.07 82.01) (end 128.109998 82.01) (width 0.5) (layer F.Cu) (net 11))
 (segment (start 131.689999 85.590001) (end 131.689999 92.410001) (width 0.5) (layer F.Cu) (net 11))
 (segment (start 132.2578 75.368) (end 130.715801 76.909999) (width 0.5) (layer F.Cu) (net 11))
 (segment (start 130.715801 76.909999) (end 129.939999 76.909999) (width 0.5) (layer F.Cu) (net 11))
 (segment (start 129.939999 76.909999) (end 129.869999 76.979999) (width 0.5) (layer F.Cu) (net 11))
 (segment (start 129.869999 76.979999) (end 129.869999 79.340001) (width 0.5) (layer F.Cu) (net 11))
 (segment (start 129.869999 79.340001) (end 131.689999 81.160001) (width 0.5) (layer F.Cu) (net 11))
 (segment (start 131.689999 81.160001) (end 131.689999 85.590001) (width 0.5) (layer F.Cu) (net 11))
 (segment (start 115.884999 78.380001) (end 117.244998 79.74) (width 0.25) (layer B.Cu) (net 19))
 (segment (start 115.884999 73.345001) (end 115.884999 78.380001) (width 0.25) (layer B.Cu) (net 19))
 (segment (start 116.96 72.27) (end 115.884999 73.345001) (width 0.25) (layer B.Cu) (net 19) (status 10))
 (segment (start 117.244998 79.74) (end 118.11 79.74) (width 0.25) (layer B.Cu) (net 19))
 (via (at 118.11 79.74) (size 0.8) (drill 0.4) (layers F.Cu B.Cu) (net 19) (status 30))
 (segment (start 116.62 81.66) (end 118.12 81.66) (width 0.25) (layer F.Cu) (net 18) (status 20))
 (segment (start 115.884999 80.924999) (end 116.62 81.66) (width 0.25) (layer F.Cu) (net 18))
 (segment (start 115.884999 70.805001) (end 115.884999 80.924999) (width 0.25) (layer F.Cu) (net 18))
 (segment (start 116.96 69.73) (end 115.884999 70.805001) (width 0.25) (layer F.Cu) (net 18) (status 10))
 (via (at 134.493 75.63104) (size 0.8) (drill 0.4) (layers F.Cu B.Cu) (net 17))
 (segment (start 134.493 75.63104) (end 134.493 88.62568) (width 0.5) (layer B.Cu) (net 17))
 (segment (start 134.493 88.62568) (end 133.38556 89.73312) (width 0.5) (layer B.Cu) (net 17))
 (segment (start 133.38556 89.73312) (end 133.38556 89.73312) (width 0.5) (layer B.Cu) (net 17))
 (via (at 133.38556 89.73312) (size 0.8) (drill 0.4) (layers F.Cu B.Cu) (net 17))
 (segment (start 127.7874 77.0926) (end 126.72 78.16) (width 0.5) (layer F.Cu) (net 16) (status 20))
 (segment (start 127.7874 75.3488) (end 127.7874 77.0926) (width 0.5) (layer F.Cu) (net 16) (status 10))
 (segment (start 125.5268 77.3532) (end 124.72 78.16) (width 0.5) (layer F.Cu) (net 15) (status 20))
 (segment (start 125.5268 75.368) (end 125.5268 77.3532) (width 0.5) (layer F.Cu) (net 15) (status 10))
 (segment (start 119.869999 79.340001) (end 120.412998 79.883) (width 0.5) (layer F.Cu) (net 15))
 (segment (start 119.869999 74.560001) (end 119.869999 79.340001) (width 0.5) (layer F.Cu) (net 15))
 (segment (start 120.07 74.36) (end 119.869999 74.560001) (width 0.5) (layer F.Cu) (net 15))
 (segment (start 120.412998 79.883) (end 123.825 79.883) (width 0.5) (layer F.Cu) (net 15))
 (segment (start 124.72 78.988) (end 124.72 78.16) (width 0.5) (layer F.Cu) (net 15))
 (segment (start 123.825 79.883) (end 124.72 78.988) (width 0.5) (layer F.Cu) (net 15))
 (via (at 125.21 65.3) (size 0.8) (drill 0.4) (layers F.Cu B.Cu) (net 7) (status 30))
 (via (at 126.95 62.04) (size 0.8) (drill 0.4) (layers F.Cu B.Cu) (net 7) (status 30))
 (segment (start 126.95 62.04) (end 126.52 61.61) (width 0.5) (layer B.Cu) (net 7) (status 30))
 (segment (start 126.52 60.34) (end 126.6 60.26) (width 0.5) (layer B.Cu) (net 7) (status 30))
 (segment (start 126.52 61.61) (end 126.52 60.34) (width 0.5) (layer B.Cu) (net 7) (status 30))
 (segment (start 127.27 62.04) (end 128.8 60.51) (width 0.5) (layer B.Cu) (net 7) (status 30))
 (segment (start 126.95 62.04) (end 127.27 62.04) (width 0.5) (layer B.Cu) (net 7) (status 30))
 (segment (start 125.7808 63.0492) (end 126.82 62.01) (width 0.5) (layer B.Cu) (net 7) (status 30))
 (segment (start 125.7808 64.0842) (end 125.7808 63.0492) (width 0.5) (layer B.Cu) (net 7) (status 30))
 (segment (start 122.3 60.51) (end 128.8 60.51) (width 0.5) (layer F.Cu) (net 7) (status 30))
 (segment (start 132.679999 65.520001) (end 130.98 67.22) (width 0.5) (layer B.Cu) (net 2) (status 20))
 (segment (start 133.485001 65.520001) (end 132.679999 65.520001) (width 0.5) (layer B.Cu) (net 2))
 (segment (start 135.188 63.817002) (end 133.485001 65.520001) (width 0.5) (layer B.Cu) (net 2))
 (segment (start 135.188 60.69) (end 135.188 63.817002) (width 0.5) (layer B.Cu) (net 2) (status 10))
 (segment (start 130.048 75.3488) (end 128.72 76.6768) (width 0.5) (layer F.Cu) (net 14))
 (segment (start 128.72 76.6768) (end 128.72 78.16) (width 0.5) (layer F.Cu) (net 14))
 (segment (start 124.72 57.64) (end 124.7 57.66) (width 0.5) (layer B.Cu) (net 5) (status 30))
 (segment (start 124.72 55.66) (end 124.72 57.64) (width 0.5) (layer B.Cu) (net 5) (status 30))
 (via (at 124.7 57.66) (size 0.8) (drill 0.4) (layers F.Cu B.Cu) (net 5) (status 30))
 (segment (start 125.743536 70.83001) (end 126.45 70.123546) (width 0.5) (layer F.Cu) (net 5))
 (segment (start 125.534788 70.83001) (end 125.743536 70.83001) (width 0.5) (layer F.Cu) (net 5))
 (segment (start 124.137601 72.227197) (end 125.534788 70.83001) (width 0.5) (layer F.Cu) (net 5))
 (segment (start 124.137601 76.742399) (end 124.137601 72.227197) (width 0.5) (layer F.Cu) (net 5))
 (segment (start 122.72 78.16) (end 124.137601 76.742399) (width 0.5) (layer F.Cu) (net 5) (status 10))
 (segment (start 124.7 57.66) (end 124.940001 57.419999) (width 0.5) (layer F.Cu) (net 5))
 (segment (start 132.440001 57.419999) (end 133.98 58.959998) (width 0.5) (layer F.Cu) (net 5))
 (segment (start 124.940001 57.419999) (end 132.440001 57.419999) (width 0.5) (layer F.Cu) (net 5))
 (segment (start 133.98 58.959998) (end 133.98 65.76) (width 0.5) (layer F.Cu) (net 5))
 (segment (start 133.98 65.76) (end 132.2 67.54) (width 0.5) (layer F.Cu) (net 5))
 (segment (start 127.37 67.54) (end 126.45 68.46) (width 0.5) (layer F.Cu) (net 5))
 (segment (start 132.2 67.54) (end 127.37 67.54) (width 0.5) (layer F.Cu) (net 5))
 (segment (start 126.45 70.123546) (end 126.45 68.46) (width 0.5) (layer F.Cu) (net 5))
 (segment (start 123.0376 71.8749) (end 125.0825 69.83) (width 0.5) (layer F.Cu) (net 8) (status 20))
 (segment (start 123.0376 73.0188) (end 123.0376 71.8749) (width 0.5) (layer F.Cu) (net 8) (status 10))
 (segment (start 123.0376 75.8424) (end 120.72 78.16) (width 0.5) (layer F.Cu) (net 12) (status 30))
 (segment (start 123.0376 75.4188) (end 123.0376 75.8424) (width 0.5) (layer F.Cu) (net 12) (status 30))
 (segment (start 131.41 60.495) (end 131.45 60.535) (width 0.5) (layer F.Cu) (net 13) (status 30))
 (segment (start 131.41 58.52) (end 131.41 60.495) (width 0.5) (layer F.Cu) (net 13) (status 30))
 (segment (start 123.13 58.69) (end 124.7 60.26) (width 0.5) (layer B.Cu) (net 6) (status 30))
 (segment (start 122.88 58.69) (end 123.13 58.69) (width 0.5) (layer B.Cu) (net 6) (status 30))
 (segment (start 122.88 56.59) (end 122.3 56.01) (width 0.5) (layer B.Cu) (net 6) (status 30))
 (segment (start 122.88 58.69) (end 122.88 56.59) (width 0.5) (layer B.Cu) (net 6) (status 30))
 (segment (start 128.8 56.01) (end 122.3 56.01) (width 0.5) (layer F.Cu) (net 6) (status 30))
 (segment (start 128.91 56.12) (end 128.8 56.01) (width 0.5) (layer F.Cu) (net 6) (status 30))
 (segment (start 131.41 56.12) (end 128.91 56.12) (width 0.5) (layer F.Cu) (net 6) (status 30))
 (segment (start 129.59 66.25) (end 130.84 66.25) (width 0.5) (layer F.Cu) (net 10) (status 10))
 (segment (start 130.84 66.25) (end 132.9 64.19) (width 0.5) (layer F.Cu) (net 10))
 (via (at 132.9 64.19) (size 0.8) (drill 0.4) (layers F.Cu B.Cu) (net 10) (status 30))
 (via (at 130.96 64.92) (size 0.8) (drill 0.4) (layers F.Cu B.Cu) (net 1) (status 30))
 (segment (start 130.98 61.354) (end 130.98 64.17) (width 0.5) (layer B.Cu) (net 1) (status 30))
 (segment (start 131.484 60.85) (end 130.98 61.354) (width 0.5) (layer B.Cu) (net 1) (status 30))
 (segment (start 129.89 63.85) (end 130.96 64.92) (width 0.5) (layer F.Cu) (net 1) (status 10))
 (segment (start 129.59 63.85) (end 129.89 63.85) (width 0.5) (layer F.Cu) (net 1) (status 30))
 (segment (start 128.91 64.53) (end 129.59 63.85) (width 0.5) (layer F.Cu) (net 1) (status 30))
 (segment (start 127.21 64.53) (end 128.91 64.53) (width 0.5) (layer F.Cu) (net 1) (status 30))
 (segment (start 128.458011 58.170009) (end 125.774996 58.170009) (width 0.5) (layer F.Cu) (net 3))
 (via (at 125.774996 58.170009) (size 0.8) (drill 0.4) (layers F.Cu B.Cu) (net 3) (status 30))
 (segment (start 125.21 63.58) (end 127.728002 63.58) (width 0.5) (layer F.Cu) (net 3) (status 10))
 (segment (start 127.728002 63.58) (end 130.150001 61.158001) (width 0.5) (layer F.Cu) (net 3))
 (segment (start 130.150001 61.158001) (end 130.150001 59.861999) (width 0.5) (layer F.Cu) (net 3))
 (segment (start 130.150001 59.861999) (end 128.458011 58.170009) (width 0.5) (layer F.Cu) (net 3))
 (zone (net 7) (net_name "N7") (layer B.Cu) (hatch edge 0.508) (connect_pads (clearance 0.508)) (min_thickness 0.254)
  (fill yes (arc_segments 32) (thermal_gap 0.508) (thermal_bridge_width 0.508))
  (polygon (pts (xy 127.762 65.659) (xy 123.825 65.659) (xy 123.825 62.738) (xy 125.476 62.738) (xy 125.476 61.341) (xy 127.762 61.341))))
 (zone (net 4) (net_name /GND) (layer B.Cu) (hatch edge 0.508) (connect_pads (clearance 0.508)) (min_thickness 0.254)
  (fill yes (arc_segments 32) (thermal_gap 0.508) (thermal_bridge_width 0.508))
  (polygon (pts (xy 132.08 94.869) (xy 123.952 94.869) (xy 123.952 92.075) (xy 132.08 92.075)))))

